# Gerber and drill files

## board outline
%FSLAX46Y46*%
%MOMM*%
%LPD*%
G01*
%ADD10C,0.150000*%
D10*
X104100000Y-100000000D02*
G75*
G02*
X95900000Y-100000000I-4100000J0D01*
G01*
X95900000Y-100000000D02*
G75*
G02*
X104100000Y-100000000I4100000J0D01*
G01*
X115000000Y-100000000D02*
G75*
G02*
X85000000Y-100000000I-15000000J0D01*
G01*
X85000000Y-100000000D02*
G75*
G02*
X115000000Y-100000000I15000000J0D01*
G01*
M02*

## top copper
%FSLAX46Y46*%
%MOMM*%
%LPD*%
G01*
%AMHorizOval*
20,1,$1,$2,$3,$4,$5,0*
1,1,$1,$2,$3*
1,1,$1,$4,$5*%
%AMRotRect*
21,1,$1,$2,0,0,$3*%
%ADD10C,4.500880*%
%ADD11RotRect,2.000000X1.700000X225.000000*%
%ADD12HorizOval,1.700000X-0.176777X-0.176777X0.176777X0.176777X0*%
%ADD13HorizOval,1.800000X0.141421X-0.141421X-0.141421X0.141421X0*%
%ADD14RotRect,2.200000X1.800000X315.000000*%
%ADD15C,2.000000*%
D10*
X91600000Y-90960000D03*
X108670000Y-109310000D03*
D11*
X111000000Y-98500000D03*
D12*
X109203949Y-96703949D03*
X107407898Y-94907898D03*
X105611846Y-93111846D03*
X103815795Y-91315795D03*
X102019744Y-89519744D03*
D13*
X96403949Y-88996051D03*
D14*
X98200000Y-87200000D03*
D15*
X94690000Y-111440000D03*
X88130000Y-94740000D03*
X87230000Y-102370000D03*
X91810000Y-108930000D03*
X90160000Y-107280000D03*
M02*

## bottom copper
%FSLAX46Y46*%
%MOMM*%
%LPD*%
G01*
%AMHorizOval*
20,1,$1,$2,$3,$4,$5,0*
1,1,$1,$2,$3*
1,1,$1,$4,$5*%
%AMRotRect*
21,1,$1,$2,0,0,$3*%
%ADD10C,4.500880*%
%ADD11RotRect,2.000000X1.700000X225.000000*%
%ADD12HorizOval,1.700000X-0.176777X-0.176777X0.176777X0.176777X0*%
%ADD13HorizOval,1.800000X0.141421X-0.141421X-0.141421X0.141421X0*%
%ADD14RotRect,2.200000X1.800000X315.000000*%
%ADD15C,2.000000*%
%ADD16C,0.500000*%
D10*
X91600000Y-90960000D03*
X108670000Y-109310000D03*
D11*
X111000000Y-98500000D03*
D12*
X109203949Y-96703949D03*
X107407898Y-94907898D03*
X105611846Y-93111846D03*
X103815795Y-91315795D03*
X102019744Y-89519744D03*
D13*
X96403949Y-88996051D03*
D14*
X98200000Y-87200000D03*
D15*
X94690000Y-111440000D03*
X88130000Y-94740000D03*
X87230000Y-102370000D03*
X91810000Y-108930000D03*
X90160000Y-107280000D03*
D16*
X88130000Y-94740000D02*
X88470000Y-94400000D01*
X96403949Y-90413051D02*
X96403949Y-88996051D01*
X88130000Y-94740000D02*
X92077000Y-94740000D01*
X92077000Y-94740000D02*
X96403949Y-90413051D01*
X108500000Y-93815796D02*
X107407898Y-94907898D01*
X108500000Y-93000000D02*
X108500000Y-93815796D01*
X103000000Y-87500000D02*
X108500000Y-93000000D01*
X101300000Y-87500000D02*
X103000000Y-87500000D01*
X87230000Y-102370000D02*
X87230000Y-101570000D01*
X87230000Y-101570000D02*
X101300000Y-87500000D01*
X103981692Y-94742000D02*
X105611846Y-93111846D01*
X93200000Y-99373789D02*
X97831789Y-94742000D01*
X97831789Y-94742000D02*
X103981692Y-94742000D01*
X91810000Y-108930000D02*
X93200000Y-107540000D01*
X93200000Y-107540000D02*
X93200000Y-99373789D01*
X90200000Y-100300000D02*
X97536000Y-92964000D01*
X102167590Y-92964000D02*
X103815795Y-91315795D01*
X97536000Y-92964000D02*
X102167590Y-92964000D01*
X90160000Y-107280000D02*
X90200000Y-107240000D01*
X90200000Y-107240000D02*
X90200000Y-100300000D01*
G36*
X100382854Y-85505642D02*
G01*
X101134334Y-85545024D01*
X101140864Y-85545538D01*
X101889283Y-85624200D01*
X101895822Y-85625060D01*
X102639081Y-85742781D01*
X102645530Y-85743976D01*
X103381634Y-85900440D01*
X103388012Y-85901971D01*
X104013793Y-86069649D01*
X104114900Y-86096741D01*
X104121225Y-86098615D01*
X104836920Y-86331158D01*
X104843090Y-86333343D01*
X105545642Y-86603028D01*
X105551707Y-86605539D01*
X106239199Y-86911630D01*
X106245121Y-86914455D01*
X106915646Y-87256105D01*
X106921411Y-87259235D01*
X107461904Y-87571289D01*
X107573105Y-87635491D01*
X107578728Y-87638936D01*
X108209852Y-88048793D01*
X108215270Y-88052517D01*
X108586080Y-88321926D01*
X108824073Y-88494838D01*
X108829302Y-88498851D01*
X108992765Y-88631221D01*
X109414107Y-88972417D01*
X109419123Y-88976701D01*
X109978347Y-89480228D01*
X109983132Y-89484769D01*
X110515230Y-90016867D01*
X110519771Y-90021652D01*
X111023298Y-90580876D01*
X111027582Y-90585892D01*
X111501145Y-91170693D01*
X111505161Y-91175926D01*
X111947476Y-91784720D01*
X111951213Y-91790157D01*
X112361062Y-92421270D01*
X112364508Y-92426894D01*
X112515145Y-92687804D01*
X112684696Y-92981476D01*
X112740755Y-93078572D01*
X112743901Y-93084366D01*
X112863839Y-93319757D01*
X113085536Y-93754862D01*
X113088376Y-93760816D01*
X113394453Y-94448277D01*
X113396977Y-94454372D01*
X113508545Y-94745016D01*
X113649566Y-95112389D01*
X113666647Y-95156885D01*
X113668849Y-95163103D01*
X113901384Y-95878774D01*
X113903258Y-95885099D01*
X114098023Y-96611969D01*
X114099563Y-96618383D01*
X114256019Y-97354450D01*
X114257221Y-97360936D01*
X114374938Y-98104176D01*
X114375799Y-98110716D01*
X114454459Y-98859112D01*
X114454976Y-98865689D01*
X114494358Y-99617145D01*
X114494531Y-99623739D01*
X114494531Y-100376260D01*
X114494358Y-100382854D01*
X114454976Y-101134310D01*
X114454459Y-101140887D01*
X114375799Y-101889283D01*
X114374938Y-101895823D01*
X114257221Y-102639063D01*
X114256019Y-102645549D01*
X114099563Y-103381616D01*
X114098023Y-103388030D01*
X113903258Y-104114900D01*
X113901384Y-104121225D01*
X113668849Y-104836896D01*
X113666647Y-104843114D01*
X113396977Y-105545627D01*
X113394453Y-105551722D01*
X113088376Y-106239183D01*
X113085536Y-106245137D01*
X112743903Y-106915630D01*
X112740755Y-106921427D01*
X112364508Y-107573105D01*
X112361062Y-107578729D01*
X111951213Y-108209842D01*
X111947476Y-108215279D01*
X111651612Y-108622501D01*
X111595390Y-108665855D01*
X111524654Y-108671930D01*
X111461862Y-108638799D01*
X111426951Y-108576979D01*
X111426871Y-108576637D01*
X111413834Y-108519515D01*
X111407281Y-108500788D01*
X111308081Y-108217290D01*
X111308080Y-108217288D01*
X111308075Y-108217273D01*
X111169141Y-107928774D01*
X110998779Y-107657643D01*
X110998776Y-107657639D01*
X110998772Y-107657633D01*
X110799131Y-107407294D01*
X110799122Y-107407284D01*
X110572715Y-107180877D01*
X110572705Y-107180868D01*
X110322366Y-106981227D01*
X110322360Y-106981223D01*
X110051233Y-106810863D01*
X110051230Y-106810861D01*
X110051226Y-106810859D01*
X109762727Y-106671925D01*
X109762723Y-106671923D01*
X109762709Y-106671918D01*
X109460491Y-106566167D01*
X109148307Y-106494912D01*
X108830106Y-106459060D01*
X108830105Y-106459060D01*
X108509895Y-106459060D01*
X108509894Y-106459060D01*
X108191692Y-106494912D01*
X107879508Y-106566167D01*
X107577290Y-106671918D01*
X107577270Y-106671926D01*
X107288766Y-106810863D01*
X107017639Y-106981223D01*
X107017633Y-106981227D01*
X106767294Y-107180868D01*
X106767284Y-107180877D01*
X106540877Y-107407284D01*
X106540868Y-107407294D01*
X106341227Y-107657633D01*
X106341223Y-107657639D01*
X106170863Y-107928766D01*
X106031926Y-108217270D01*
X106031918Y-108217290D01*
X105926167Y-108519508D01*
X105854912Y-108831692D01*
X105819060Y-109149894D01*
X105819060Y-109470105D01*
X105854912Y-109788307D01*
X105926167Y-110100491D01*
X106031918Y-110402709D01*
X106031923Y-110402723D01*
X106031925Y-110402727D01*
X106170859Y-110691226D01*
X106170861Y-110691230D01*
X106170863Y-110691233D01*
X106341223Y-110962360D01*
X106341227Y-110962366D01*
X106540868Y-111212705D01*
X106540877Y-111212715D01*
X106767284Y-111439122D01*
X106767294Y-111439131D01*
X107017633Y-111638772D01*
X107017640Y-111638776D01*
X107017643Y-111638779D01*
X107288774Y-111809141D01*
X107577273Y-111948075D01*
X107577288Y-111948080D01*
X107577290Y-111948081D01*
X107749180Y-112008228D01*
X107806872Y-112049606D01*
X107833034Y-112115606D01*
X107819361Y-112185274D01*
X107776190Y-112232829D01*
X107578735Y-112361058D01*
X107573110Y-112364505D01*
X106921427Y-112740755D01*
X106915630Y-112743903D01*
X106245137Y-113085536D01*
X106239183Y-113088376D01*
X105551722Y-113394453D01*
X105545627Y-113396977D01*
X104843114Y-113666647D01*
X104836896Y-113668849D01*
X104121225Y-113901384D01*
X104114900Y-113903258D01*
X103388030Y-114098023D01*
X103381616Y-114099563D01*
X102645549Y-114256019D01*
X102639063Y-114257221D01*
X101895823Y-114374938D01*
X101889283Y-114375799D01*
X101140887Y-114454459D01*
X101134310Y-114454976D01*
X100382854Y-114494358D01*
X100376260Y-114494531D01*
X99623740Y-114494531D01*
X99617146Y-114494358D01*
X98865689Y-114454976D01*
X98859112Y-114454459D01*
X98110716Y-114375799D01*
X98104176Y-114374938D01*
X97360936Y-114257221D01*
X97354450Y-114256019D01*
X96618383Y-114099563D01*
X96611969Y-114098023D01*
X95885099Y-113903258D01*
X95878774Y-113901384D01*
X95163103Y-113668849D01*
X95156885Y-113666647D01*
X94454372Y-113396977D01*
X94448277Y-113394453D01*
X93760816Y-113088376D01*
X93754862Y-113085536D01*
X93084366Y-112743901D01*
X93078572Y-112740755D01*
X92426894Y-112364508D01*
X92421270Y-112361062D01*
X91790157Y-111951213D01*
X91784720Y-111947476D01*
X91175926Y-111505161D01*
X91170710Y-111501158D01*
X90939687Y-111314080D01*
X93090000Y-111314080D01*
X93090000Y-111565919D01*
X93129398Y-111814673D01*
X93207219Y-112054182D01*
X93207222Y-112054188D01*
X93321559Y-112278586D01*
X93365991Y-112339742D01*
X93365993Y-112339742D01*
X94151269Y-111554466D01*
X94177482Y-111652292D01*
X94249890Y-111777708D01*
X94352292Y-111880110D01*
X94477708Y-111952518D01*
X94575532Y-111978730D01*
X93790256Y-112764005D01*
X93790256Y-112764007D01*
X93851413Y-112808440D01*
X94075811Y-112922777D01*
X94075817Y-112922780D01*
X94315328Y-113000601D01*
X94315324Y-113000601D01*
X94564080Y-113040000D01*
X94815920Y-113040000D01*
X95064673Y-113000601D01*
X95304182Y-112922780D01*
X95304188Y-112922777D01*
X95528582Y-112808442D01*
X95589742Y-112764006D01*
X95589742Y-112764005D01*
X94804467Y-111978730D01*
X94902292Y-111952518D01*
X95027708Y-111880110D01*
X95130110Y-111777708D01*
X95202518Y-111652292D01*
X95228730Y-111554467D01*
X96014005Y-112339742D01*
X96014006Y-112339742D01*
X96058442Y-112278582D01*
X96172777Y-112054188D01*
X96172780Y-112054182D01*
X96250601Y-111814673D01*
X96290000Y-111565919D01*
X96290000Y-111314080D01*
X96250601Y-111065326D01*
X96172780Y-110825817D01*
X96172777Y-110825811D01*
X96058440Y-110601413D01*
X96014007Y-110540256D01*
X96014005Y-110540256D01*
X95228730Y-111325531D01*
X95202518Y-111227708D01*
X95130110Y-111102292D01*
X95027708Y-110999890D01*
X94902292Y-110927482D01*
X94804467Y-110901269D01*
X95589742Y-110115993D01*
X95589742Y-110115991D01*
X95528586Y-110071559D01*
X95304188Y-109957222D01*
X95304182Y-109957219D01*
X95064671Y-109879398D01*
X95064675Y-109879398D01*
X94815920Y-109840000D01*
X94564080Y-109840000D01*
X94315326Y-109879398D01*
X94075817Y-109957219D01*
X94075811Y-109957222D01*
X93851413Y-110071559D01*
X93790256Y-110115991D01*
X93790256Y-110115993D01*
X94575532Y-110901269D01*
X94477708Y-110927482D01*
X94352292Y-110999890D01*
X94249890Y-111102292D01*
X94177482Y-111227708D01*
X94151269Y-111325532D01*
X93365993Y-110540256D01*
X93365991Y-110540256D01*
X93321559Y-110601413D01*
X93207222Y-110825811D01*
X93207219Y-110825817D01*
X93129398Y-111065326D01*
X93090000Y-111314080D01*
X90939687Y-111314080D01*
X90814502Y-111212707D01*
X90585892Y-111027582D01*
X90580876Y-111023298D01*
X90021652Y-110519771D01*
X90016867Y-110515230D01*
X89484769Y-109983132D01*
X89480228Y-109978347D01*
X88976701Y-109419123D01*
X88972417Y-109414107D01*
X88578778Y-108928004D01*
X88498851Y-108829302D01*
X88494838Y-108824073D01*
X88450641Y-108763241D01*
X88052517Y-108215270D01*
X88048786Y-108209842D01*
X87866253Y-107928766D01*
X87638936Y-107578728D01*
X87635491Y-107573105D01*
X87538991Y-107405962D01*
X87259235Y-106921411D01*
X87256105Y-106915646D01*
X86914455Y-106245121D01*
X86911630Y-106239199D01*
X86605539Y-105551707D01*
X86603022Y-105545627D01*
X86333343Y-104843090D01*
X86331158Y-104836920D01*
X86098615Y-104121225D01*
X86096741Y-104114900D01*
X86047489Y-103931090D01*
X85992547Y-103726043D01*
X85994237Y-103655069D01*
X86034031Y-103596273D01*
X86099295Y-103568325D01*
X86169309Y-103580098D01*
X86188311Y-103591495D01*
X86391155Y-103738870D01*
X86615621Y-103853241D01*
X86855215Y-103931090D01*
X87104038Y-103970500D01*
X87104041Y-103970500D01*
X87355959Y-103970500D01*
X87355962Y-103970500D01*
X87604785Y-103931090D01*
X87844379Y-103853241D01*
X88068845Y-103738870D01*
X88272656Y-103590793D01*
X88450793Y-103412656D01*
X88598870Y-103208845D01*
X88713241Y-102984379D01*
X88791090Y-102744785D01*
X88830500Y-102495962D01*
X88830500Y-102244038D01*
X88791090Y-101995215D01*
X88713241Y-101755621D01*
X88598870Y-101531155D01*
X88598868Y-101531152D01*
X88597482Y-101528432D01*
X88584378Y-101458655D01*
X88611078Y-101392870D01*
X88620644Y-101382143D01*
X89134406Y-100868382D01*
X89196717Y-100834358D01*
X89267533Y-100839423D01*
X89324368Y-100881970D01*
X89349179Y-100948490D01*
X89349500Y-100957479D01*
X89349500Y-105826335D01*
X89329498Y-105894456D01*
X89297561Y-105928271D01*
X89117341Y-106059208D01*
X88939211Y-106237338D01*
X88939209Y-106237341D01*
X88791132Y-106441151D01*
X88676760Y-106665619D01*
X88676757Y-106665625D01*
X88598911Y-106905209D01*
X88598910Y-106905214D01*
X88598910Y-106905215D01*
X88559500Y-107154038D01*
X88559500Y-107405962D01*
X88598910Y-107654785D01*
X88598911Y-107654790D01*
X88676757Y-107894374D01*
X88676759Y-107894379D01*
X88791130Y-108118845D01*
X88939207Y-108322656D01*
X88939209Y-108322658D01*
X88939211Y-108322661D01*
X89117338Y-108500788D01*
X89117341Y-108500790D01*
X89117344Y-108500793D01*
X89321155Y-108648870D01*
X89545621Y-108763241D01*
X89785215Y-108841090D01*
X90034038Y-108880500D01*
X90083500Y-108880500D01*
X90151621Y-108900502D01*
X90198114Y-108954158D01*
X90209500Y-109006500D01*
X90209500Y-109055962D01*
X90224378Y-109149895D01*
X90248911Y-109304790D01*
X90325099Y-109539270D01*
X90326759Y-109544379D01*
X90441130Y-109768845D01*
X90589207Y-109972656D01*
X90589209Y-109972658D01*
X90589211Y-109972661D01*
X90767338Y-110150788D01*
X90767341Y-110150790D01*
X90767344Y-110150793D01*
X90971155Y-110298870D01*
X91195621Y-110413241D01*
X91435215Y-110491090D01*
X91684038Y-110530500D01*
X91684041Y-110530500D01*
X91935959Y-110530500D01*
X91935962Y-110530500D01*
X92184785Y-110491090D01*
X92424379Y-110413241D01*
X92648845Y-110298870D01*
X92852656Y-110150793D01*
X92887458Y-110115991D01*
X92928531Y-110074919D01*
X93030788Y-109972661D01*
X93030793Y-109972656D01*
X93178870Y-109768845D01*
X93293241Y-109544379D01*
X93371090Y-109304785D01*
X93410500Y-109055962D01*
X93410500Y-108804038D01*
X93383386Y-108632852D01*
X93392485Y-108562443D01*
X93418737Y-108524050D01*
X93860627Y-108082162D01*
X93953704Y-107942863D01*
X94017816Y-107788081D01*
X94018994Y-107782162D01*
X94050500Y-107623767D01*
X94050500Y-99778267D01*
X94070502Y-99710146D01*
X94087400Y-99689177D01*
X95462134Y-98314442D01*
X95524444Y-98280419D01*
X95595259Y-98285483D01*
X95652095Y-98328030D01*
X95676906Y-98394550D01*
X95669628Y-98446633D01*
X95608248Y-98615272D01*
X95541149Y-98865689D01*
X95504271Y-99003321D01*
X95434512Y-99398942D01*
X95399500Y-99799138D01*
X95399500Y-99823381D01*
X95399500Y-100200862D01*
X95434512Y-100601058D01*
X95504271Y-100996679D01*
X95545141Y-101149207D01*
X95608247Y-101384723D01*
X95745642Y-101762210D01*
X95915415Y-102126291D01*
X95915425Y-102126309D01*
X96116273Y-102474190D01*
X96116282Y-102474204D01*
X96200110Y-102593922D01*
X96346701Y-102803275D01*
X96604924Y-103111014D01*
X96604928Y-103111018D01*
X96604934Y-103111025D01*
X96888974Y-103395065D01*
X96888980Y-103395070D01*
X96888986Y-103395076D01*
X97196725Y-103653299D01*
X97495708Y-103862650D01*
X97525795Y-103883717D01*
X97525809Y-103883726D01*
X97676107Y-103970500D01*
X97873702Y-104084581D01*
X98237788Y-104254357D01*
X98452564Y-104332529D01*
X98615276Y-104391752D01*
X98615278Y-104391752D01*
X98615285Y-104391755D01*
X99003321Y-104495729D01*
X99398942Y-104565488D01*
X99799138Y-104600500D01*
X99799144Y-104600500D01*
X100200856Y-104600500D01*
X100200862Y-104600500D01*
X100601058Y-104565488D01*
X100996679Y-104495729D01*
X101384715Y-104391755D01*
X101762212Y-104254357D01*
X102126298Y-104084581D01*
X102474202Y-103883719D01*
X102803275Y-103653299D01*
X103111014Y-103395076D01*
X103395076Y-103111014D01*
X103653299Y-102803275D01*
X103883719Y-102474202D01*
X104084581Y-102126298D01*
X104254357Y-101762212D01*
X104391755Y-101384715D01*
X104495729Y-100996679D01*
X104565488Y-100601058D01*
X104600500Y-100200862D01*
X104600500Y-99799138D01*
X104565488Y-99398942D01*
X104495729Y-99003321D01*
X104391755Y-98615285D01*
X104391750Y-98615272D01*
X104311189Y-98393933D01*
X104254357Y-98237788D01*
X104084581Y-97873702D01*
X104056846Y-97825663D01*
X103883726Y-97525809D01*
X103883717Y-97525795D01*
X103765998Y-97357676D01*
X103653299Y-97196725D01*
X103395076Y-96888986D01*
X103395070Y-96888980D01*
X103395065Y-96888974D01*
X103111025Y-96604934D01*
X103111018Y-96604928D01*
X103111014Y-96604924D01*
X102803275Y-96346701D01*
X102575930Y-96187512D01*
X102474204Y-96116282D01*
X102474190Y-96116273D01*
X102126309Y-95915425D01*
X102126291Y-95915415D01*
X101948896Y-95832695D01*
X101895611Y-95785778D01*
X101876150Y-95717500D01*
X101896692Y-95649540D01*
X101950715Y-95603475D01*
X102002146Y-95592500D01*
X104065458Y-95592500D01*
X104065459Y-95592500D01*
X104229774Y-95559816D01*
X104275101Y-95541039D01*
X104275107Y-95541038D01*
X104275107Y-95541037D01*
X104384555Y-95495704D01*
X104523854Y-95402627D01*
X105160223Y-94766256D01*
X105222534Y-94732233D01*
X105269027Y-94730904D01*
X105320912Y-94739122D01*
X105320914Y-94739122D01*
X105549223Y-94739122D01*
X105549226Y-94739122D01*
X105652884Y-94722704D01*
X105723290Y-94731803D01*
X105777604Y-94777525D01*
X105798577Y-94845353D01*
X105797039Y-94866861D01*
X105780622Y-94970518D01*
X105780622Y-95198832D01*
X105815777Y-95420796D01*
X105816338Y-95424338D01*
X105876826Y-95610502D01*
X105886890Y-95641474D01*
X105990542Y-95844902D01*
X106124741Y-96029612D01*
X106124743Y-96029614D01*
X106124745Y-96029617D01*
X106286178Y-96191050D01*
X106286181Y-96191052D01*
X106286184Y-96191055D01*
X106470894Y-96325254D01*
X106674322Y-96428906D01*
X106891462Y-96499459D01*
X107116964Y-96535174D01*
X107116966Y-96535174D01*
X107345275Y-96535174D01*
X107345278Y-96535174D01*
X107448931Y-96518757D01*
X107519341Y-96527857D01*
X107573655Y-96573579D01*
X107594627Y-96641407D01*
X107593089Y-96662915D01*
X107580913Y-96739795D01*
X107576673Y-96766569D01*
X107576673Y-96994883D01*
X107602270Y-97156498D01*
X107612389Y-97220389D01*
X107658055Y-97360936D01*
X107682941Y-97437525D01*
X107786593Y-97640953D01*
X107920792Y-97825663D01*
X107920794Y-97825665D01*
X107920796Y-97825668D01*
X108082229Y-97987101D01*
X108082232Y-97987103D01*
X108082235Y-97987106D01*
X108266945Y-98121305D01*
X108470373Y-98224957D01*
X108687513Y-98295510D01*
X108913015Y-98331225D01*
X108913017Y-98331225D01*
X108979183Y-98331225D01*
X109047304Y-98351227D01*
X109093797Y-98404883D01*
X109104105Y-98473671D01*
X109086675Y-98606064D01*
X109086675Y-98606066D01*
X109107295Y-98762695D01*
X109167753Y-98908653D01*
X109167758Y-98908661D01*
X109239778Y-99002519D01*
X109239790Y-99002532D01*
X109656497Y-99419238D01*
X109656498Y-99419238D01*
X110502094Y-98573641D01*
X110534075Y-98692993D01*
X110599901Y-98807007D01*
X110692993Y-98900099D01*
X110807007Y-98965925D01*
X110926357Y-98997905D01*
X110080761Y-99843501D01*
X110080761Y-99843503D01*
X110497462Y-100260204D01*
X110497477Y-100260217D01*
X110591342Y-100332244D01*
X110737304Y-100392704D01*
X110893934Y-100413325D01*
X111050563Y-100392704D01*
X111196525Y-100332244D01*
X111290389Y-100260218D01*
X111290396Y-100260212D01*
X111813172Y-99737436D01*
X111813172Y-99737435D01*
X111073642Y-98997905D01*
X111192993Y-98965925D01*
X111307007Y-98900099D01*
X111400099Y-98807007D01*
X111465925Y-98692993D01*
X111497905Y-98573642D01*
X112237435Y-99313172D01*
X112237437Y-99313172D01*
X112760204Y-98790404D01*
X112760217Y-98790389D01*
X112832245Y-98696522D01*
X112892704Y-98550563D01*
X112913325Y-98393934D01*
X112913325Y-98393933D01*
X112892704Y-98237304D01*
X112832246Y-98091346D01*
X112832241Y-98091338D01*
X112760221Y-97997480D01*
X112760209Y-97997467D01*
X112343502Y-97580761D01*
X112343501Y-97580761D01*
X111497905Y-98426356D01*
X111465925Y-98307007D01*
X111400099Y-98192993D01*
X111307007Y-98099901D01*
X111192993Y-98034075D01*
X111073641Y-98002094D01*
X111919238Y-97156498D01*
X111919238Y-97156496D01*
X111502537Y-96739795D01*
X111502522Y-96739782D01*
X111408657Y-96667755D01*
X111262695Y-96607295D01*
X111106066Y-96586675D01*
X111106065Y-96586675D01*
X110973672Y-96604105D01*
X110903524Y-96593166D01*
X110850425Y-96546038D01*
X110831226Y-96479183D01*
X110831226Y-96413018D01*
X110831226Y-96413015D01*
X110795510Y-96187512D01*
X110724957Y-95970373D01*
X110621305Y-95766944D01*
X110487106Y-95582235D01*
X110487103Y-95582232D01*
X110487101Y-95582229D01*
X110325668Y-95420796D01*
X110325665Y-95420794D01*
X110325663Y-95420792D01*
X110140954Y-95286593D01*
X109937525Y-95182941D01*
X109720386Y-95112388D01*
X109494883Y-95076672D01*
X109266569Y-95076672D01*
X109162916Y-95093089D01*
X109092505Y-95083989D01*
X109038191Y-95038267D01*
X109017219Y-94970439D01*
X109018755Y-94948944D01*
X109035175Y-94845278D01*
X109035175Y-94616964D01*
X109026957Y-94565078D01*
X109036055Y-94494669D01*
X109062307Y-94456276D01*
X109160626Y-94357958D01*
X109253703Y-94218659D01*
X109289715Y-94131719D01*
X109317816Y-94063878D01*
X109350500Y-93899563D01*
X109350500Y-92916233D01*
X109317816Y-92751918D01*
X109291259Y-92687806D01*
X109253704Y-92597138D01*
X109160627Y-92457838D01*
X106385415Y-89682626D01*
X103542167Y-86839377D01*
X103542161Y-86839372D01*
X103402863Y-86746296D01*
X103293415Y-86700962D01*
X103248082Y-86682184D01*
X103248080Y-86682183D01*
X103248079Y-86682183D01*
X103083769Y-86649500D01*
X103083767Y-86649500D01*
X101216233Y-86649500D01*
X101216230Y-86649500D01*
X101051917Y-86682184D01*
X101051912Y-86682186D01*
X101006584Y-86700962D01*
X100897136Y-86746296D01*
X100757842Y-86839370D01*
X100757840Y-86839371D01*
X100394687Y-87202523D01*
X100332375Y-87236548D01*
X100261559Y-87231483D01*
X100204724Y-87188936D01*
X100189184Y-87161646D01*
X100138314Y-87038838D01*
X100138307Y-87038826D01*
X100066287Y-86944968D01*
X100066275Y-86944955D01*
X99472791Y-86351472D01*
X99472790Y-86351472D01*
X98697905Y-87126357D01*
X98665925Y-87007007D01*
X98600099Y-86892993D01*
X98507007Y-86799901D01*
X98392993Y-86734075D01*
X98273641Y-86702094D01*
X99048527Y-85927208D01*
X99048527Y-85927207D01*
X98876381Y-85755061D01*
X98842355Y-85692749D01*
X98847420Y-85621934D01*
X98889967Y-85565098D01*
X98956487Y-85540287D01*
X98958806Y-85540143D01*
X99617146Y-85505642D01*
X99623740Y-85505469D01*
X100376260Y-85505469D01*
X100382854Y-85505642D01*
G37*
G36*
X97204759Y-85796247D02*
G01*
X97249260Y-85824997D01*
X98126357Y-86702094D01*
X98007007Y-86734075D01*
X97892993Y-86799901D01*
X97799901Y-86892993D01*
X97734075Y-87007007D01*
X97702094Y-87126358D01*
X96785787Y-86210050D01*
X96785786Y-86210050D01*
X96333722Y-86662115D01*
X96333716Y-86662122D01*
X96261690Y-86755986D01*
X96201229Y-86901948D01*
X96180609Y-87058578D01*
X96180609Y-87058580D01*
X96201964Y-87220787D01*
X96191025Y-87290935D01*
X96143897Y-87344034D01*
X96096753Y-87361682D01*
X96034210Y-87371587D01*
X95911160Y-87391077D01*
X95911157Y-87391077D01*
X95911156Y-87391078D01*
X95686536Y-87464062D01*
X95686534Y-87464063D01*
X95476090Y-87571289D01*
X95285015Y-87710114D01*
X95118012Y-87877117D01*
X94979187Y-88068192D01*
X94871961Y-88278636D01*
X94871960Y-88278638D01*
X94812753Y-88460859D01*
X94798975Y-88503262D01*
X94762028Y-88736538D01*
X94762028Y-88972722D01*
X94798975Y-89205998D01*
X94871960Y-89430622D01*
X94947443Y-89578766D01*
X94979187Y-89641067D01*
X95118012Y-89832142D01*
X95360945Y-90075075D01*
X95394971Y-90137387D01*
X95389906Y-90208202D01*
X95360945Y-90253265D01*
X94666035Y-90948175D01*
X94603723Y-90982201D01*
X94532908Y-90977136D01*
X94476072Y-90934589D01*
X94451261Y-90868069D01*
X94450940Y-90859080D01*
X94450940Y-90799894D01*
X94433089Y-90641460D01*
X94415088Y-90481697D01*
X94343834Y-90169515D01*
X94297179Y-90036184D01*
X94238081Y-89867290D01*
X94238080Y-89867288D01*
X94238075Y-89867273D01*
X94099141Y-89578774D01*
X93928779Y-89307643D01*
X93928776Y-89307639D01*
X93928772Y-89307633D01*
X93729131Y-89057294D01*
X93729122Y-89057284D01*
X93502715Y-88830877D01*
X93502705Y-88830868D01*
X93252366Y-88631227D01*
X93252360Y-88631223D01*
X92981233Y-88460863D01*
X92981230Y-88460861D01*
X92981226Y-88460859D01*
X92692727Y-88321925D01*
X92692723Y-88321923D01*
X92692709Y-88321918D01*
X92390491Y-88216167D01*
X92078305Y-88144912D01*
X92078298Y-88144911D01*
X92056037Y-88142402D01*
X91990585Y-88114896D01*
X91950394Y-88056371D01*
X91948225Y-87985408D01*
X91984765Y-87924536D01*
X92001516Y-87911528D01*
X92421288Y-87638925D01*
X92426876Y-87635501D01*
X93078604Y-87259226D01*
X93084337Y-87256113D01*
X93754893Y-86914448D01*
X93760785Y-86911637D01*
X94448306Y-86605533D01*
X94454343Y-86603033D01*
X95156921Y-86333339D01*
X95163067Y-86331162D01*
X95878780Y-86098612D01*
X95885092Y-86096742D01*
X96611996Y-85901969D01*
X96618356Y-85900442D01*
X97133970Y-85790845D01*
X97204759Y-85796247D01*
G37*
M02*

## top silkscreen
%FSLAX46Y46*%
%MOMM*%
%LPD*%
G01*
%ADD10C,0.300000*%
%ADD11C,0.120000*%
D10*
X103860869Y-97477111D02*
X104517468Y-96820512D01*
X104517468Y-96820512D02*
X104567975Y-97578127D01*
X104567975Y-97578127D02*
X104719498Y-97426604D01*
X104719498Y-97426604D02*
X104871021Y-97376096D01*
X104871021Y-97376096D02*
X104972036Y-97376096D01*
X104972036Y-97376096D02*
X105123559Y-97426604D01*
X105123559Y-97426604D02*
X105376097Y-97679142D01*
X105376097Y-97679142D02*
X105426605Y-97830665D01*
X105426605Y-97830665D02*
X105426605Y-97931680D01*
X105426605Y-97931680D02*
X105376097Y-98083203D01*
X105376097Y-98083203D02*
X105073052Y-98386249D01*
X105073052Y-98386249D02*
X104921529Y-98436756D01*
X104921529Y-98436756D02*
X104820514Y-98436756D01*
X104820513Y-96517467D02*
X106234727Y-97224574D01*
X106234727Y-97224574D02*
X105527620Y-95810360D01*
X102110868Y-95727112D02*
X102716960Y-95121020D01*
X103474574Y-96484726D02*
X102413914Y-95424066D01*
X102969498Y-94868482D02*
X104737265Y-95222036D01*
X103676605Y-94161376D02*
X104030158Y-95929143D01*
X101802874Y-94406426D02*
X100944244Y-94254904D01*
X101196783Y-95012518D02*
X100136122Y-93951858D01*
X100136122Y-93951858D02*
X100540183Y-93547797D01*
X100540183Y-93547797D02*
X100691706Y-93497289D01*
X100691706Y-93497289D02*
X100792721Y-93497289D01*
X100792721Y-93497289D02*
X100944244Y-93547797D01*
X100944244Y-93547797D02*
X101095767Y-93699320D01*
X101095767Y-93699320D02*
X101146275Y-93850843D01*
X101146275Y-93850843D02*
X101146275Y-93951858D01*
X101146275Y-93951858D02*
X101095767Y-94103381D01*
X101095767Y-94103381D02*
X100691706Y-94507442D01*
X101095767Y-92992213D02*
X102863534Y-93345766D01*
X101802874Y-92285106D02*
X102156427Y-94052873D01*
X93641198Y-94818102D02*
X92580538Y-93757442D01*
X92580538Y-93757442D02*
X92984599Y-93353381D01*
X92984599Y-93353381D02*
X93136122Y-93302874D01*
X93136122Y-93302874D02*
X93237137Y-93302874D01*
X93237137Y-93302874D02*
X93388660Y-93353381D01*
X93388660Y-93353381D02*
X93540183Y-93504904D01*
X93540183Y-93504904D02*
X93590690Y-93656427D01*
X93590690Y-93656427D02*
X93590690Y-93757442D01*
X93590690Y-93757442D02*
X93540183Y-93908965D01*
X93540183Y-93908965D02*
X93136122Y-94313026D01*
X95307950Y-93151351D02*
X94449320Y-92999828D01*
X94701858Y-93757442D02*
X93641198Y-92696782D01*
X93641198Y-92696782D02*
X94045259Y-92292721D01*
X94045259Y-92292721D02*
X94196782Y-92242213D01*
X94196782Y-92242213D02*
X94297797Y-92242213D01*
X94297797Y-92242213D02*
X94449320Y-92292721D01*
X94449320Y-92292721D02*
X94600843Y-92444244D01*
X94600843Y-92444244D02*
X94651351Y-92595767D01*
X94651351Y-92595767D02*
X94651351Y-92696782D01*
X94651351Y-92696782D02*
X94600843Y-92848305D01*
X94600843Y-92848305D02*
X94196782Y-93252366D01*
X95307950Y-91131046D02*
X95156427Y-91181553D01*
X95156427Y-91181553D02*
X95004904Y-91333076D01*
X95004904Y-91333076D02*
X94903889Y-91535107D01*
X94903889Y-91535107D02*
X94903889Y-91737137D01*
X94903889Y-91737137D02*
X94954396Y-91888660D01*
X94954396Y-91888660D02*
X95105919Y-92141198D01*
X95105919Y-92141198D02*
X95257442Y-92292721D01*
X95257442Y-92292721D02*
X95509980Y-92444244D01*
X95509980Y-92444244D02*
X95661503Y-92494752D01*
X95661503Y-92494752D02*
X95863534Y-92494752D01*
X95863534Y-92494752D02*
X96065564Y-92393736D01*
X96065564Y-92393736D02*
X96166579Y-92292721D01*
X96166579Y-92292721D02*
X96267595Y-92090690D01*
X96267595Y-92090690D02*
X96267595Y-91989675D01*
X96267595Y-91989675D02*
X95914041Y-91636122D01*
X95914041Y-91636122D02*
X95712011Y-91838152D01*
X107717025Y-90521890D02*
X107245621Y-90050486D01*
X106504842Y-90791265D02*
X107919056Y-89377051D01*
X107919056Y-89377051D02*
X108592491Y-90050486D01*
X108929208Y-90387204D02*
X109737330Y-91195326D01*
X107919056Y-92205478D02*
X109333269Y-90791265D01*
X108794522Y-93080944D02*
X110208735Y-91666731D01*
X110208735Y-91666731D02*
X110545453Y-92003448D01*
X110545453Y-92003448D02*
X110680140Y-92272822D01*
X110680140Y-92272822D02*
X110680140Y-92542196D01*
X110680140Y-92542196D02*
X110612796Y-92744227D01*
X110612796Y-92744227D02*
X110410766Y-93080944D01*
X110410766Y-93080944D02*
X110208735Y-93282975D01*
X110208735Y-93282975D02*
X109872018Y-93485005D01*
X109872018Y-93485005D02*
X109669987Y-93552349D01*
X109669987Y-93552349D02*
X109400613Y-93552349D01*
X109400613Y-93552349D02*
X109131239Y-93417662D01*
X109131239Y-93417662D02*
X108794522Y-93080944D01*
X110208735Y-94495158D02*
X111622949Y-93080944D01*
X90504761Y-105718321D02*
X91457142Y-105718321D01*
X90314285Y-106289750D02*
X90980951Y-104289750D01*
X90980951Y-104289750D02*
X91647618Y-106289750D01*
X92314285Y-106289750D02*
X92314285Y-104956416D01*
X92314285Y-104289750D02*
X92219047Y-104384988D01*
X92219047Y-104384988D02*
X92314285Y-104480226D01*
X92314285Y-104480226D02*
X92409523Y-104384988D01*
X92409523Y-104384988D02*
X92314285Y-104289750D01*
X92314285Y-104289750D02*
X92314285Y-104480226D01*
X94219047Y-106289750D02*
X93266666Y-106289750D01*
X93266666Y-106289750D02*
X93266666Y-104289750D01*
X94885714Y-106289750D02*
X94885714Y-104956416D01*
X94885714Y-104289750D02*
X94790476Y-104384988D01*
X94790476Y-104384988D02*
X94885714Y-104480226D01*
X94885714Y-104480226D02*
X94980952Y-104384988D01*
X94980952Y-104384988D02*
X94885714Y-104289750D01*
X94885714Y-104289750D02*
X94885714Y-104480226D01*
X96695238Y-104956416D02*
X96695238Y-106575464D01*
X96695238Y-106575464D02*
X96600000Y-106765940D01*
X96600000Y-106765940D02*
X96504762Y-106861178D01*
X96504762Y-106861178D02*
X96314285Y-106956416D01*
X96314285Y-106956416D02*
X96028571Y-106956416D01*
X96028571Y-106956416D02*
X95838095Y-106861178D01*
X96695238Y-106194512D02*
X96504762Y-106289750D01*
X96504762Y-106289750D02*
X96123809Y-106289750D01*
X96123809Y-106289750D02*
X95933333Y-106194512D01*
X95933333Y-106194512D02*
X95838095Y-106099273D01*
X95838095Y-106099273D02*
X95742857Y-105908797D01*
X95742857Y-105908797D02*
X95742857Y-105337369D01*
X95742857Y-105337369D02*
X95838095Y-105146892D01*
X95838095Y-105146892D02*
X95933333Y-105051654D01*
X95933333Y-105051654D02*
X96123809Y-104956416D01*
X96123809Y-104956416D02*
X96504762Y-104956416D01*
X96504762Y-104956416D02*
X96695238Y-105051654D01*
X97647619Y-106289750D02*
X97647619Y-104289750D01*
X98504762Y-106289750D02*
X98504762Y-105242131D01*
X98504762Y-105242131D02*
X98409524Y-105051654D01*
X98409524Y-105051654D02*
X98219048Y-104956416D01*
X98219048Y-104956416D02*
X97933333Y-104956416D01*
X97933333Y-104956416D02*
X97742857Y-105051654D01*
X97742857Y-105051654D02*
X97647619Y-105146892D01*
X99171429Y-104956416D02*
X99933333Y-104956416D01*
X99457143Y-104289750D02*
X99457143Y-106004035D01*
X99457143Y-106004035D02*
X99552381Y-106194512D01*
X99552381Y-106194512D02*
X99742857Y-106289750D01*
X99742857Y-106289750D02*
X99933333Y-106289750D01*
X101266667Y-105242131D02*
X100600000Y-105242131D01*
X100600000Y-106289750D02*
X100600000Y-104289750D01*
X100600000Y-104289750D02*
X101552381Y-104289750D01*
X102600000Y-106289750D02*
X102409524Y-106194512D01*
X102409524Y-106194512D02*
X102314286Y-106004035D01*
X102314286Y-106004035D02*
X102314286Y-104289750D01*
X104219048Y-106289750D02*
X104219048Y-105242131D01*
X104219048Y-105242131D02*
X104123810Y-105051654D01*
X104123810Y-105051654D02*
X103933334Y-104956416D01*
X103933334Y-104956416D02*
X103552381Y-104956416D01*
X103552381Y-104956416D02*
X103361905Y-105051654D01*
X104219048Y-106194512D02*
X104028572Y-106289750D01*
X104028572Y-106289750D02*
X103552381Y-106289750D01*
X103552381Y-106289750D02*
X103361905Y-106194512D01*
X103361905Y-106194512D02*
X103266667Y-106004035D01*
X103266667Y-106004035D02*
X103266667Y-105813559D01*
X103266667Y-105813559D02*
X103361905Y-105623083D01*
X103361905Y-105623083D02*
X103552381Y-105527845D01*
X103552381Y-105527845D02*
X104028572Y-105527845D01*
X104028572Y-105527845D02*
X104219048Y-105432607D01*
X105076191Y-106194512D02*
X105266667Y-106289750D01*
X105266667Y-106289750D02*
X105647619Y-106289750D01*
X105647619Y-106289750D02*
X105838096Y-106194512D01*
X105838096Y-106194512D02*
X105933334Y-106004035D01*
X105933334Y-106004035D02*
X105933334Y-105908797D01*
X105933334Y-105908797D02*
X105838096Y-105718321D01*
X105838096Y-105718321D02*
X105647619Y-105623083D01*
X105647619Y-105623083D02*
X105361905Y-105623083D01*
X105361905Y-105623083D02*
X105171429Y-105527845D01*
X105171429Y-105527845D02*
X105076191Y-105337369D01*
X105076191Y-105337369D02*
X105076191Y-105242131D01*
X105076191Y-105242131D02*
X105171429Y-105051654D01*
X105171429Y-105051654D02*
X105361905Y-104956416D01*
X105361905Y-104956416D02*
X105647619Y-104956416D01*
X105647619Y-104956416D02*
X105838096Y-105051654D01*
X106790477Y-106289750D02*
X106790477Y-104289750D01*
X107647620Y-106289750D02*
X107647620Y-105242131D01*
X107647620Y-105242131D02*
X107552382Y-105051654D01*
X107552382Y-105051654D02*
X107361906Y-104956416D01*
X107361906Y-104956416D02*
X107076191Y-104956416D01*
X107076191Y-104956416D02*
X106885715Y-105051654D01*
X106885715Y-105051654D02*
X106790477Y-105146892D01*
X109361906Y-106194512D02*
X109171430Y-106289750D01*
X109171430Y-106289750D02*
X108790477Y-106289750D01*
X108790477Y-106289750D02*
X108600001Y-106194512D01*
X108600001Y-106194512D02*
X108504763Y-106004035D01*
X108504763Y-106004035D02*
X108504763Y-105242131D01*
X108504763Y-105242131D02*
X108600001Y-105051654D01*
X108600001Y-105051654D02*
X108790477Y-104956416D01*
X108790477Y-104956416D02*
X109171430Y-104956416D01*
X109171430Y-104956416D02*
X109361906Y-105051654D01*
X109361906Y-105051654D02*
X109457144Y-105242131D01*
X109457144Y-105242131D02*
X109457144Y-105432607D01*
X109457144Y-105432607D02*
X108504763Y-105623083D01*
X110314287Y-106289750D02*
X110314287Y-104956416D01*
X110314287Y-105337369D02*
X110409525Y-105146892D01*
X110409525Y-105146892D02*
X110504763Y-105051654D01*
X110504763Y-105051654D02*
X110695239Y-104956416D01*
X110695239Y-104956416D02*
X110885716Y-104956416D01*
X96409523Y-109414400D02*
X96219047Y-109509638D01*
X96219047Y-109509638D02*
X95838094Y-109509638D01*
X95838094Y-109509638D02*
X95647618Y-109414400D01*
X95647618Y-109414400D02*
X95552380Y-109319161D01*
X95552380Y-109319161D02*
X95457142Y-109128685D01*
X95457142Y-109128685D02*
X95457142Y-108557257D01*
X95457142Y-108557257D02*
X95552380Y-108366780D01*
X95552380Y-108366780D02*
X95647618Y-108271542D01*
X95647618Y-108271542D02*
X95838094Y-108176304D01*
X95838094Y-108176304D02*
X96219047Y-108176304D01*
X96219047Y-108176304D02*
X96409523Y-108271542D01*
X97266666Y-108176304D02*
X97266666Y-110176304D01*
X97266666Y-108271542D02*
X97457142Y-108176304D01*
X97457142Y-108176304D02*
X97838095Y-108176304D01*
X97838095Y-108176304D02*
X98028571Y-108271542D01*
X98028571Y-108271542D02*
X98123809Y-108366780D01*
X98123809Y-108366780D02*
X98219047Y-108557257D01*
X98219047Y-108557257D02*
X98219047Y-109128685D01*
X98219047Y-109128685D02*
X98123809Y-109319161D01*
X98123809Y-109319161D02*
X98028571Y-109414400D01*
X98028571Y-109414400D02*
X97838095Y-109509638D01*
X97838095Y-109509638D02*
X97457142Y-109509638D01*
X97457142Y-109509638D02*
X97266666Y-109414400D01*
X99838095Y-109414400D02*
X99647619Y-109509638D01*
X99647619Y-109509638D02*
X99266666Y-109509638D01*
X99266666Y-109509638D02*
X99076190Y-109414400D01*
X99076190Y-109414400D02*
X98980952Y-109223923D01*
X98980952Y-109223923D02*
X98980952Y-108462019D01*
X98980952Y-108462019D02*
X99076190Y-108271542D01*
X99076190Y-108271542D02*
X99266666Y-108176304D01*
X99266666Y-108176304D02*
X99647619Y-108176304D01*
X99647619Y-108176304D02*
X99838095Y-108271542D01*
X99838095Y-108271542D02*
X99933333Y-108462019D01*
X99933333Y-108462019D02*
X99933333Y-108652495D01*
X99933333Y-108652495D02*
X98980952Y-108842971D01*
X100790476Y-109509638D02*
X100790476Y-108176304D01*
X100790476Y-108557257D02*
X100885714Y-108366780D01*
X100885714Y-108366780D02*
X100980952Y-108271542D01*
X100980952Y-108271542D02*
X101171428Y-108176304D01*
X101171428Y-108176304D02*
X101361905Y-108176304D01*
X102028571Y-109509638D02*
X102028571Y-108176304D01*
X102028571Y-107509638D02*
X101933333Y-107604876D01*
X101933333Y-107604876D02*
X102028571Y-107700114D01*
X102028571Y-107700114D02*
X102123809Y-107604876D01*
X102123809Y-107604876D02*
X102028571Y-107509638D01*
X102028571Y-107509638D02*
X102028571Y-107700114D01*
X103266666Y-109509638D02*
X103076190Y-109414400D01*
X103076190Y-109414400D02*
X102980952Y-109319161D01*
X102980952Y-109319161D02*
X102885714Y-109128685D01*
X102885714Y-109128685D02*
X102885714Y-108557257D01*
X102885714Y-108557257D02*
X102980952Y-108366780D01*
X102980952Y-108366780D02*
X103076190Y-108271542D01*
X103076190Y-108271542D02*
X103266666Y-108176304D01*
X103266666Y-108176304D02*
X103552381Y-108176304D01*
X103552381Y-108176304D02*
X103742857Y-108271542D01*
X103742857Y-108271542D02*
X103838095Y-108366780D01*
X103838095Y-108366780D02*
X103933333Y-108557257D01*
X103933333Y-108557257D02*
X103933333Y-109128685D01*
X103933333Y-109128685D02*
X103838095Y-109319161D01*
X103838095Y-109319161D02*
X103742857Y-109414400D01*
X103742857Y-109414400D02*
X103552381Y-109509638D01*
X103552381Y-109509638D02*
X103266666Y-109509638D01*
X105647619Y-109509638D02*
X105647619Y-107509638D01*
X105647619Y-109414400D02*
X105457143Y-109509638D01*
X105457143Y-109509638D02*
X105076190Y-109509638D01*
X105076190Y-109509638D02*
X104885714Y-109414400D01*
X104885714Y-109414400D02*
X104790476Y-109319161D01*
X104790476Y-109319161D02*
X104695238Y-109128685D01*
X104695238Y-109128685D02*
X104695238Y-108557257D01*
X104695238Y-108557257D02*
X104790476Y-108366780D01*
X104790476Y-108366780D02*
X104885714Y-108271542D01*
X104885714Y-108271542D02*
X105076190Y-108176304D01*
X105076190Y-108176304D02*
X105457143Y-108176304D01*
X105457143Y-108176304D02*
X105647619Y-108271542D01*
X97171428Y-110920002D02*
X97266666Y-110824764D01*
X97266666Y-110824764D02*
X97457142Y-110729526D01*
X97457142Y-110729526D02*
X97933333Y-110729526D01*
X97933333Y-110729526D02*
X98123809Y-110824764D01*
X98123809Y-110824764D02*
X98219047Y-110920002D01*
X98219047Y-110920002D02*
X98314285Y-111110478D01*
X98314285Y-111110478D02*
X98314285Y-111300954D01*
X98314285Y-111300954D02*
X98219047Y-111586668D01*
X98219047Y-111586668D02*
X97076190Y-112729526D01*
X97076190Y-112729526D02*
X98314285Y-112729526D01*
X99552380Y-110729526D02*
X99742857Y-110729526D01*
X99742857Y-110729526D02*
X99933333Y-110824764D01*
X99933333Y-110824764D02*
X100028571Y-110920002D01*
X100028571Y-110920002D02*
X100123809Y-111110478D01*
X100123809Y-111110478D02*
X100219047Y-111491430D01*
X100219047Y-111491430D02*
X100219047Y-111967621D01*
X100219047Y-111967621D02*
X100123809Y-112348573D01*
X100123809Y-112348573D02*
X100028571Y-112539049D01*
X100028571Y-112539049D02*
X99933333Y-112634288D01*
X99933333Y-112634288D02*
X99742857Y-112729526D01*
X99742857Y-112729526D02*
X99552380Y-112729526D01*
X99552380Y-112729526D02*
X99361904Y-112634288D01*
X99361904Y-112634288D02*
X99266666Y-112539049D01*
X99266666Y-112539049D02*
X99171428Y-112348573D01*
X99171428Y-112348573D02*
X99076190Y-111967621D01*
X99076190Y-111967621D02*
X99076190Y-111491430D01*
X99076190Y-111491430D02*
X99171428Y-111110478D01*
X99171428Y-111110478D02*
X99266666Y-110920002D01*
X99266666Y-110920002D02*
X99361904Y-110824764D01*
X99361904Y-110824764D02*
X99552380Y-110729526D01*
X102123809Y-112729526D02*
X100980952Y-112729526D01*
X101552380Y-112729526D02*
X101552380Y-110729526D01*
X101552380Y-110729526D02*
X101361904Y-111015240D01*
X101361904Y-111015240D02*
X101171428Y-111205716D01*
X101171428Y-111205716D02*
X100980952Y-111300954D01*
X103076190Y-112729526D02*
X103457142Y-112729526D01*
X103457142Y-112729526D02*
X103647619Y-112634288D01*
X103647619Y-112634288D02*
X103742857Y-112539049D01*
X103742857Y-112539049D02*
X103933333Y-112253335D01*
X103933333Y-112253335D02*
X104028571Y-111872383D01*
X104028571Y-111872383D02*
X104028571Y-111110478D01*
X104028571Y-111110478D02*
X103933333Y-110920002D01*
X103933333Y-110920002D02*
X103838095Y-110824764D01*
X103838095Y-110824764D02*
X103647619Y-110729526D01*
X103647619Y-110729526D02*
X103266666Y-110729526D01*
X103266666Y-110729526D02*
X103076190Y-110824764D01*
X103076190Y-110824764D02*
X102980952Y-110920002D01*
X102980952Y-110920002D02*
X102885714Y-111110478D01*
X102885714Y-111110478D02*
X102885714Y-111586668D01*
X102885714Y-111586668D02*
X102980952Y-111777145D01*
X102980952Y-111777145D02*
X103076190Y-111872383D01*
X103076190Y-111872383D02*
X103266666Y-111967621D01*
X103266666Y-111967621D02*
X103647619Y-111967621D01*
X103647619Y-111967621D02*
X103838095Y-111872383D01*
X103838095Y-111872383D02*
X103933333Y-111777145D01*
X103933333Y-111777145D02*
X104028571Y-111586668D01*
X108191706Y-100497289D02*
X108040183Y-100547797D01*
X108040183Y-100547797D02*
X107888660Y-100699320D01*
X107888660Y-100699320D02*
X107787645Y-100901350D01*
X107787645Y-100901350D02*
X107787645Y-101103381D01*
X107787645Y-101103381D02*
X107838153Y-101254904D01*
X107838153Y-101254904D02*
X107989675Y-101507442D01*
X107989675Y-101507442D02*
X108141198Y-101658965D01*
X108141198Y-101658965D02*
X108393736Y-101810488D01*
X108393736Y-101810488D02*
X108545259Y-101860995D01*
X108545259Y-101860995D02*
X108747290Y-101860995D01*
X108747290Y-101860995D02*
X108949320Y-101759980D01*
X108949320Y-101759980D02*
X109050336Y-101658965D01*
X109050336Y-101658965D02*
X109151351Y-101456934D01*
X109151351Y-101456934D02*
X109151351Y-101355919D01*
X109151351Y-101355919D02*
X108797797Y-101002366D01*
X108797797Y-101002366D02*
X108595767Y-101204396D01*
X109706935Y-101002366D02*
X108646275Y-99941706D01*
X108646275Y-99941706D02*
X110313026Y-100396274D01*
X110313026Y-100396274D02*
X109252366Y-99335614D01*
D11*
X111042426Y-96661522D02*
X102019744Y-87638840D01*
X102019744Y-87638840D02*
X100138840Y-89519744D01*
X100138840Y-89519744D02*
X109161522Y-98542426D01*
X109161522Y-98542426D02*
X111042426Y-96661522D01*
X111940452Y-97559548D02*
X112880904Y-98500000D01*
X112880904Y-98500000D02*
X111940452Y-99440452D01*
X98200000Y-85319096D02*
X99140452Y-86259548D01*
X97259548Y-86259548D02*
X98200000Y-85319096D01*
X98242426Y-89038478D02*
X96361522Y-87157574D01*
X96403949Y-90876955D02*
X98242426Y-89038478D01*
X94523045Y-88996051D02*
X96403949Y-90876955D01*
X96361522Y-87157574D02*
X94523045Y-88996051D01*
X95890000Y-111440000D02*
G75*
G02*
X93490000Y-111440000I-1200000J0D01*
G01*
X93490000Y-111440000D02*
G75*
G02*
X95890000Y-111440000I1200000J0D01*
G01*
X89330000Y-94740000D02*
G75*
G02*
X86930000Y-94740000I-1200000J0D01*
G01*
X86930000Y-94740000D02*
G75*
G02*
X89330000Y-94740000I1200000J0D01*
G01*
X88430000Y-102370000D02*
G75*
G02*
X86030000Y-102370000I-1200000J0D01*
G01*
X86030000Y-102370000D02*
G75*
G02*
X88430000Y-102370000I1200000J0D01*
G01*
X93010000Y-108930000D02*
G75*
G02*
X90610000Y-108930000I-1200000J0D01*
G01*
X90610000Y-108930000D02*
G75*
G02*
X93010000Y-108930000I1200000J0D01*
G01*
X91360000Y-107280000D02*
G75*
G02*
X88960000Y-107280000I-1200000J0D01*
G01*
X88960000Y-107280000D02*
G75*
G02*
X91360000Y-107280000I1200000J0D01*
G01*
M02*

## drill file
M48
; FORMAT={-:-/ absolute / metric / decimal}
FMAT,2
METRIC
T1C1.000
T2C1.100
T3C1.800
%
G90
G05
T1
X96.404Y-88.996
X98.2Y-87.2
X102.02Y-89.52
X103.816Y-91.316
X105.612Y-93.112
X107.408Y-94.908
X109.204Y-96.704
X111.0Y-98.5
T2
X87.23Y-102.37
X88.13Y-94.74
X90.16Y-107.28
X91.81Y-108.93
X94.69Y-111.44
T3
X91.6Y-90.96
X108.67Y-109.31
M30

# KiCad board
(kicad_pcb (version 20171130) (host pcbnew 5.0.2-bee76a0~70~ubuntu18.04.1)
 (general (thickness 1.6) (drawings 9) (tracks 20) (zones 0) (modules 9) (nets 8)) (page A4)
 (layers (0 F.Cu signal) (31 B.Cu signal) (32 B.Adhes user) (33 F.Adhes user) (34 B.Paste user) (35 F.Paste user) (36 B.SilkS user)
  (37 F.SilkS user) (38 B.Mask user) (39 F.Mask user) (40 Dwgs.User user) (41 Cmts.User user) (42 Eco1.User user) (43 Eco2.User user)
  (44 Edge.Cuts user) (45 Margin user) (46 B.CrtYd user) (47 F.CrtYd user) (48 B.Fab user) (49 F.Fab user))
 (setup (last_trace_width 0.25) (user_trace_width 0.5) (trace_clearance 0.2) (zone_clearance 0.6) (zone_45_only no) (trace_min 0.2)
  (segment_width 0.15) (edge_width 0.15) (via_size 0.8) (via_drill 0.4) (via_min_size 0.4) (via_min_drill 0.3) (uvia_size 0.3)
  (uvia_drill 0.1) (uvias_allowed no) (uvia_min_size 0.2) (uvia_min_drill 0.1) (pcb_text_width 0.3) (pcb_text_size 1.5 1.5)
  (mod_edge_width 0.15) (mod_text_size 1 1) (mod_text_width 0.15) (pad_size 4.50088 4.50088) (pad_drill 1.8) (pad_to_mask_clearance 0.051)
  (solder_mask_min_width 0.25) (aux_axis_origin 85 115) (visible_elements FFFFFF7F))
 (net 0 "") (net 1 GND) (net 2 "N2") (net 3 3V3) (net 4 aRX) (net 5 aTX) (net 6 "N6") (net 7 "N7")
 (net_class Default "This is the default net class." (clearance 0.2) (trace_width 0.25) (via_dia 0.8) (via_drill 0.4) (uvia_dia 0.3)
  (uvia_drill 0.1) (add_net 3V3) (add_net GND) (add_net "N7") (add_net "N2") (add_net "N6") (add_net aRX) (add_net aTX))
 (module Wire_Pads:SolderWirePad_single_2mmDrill (layer F.Cu) (at 91.6 90.96)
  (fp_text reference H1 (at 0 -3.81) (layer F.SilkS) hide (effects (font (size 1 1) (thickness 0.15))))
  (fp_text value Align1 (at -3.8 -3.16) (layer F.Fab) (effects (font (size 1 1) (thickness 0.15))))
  (pad 1 thru_hole circle (at 0 0) (size 4.50088 4.50088) (drill 1.8) (layers *.Cu *.Mask)))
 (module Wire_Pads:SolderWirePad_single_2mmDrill (layer F.Cu) (at 108.67 109.31)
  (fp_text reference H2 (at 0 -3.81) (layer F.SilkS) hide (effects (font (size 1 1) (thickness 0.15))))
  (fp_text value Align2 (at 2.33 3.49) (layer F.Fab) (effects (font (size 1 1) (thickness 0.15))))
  (pad 1 thru_hole circle (at 0 0) (size 4.50088 4.50088) (drill 1.8) (layers *.Cu *.Mask)))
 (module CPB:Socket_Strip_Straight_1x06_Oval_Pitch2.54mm (layer F.Cu) (at 111 98.5 225)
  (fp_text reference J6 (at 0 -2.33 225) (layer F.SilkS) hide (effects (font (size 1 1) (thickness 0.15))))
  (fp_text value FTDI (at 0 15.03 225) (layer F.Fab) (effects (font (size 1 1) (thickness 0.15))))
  (fp_line (start -1.33 1.27) (end -1.33 14.03) (layer F.SilkS) (width 0.12))
  (fp_line (start -1.33 14.03) (end 1.33 14.03) (layer F.SilkS) (width 0.12))
  (fp_line (start 1.33 14.03) (end 1.33 1.27) (layer F.SilkS) (width 0.12))
  (fp_line (start 1.33 1.27) (end -1.33 1.27) (layer F.SilkS) (width 0.12))
  (fp_line (start -1.33 0) (end -1.33 -1.33) (layer F.SilkS) (width 0.12))
  (fp_line (start -1.33 -1.33) (end 0 -1.33) (layer F.SilkS) (width 0.12))
  (pad 1 thru_hole rect (at 0 0 225) (size 2 1.7) (drill 1) (layers *.Cu *.Mask) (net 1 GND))
  (pad 2 thru_hole oval (at 0 2.54 225) (size 2.2 1.7) (drill 1) (layers *.Cu *.Mask) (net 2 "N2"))
  (pad 3 thru_hole oval (at 0 5.079999 225) (size 2.2 1.7) (drill 1) (layers *.Cu *.Mask) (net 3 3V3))
  (pad 4 thru_hole oval (at 0 7.62 225) (size 2.2 1.7) (drill 1) (layers *.Cu *.Mask) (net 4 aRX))
  (pad 5 thru_hole oval (at 0 10.16 225) (size 2.2 1.7) (drill 1) (layers *.Cu *.Mask) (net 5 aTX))
  (pad 6 thru_hole oval (at 0 12.7 225) (size 2.2 1.7) (drill 1) (layers *.Cu *.Mask) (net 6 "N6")))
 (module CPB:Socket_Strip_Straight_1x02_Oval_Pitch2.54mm (layer F.Cu) (at 98.2 87.2 315)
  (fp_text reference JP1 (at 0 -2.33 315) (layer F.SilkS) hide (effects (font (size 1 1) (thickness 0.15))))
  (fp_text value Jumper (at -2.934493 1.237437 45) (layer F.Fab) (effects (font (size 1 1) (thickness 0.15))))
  (fp_line (start -1.33 -1.33) (end 0 -1.33) (layer F.SilkS) (width 0.12))
  (fp_line (start -1.33 0) (end -1.33 -1.33) (layer F.SilkS) (width 0.12))
  (fp_line (start 1.33 1.27) (end -1.33 1.27) (layer F.SilkS) (width 0.12))
  (fp_line (start 1.33 3.87) (end 1.33 1.27) (layer F.SilkS) (width 0.12))
  (fp_line (start -1.33 3.87) (end 1.33 3.87) (layer F.SilkS) (width 0.12))
  (fp_line (start -1.33 1.27) (end -1.33 3.87) (layer F.SilkS) (width 0.12))
  (pad 2 thru_hole oval (at 0 2.54 315) (size 2.2 1.8) (drill 1) (layers *.Cu *.Mask) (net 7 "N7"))
  (pad 1 thru_hole rect (at 0 0 315) (size 2.2 1.8) (drill 1) (layers *.Cu *.Mask) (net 1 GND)))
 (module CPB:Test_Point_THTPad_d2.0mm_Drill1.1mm (layer F.Cu) (at 94.69 111.44)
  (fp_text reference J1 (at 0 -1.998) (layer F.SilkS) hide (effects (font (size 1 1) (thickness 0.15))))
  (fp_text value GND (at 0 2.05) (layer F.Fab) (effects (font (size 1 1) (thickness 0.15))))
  (fp_circle (center 0 0) (end 0 1.2) (layer F.SilkS) (width 0.12))
  (pad 1 thru_hole circle (at 0 0) (size 2 2) (drill 1.1) (layers *.Cu *.Mask) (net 1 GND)))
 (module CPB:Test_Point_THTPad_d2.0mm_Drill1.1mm (layer F.Cu) (at 88.13 94.74)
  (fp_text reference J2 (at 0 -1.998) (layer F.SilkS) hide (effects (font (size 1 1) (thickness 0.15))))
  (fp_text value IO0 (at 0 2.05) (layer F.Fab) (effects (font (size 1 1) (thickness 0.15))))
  (fp_circle (center 0 0) (end 0 1.2) (layer F.SilkS) (width 0.12))
  (pad 1 thru_hole circle (at 0 0) (size 2 2) (drill 1.1) (layers *.Cu *.Mask) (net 7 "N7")))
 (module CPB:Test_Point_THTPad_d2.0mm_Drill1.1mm (layer F.Cu) (at 87.23 102.37)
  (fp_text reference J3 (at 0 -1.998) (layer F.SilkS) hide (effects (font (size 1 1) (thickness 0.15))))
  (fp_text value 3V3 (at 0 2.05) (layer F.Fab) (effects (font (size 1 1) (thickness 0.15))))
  (fp_circle (center 0 0) (end 0 1.2) (layer F.SilkS) (width 0.12))
  (pad 1 thru_hole circle (at 0 0) (size 2 2) (drill 1.1) (layers *.Cu *.Mask) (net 3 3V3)))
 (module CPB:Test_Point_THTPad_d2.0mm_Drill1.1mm (layer F.Cu) (at 91.81 108.93)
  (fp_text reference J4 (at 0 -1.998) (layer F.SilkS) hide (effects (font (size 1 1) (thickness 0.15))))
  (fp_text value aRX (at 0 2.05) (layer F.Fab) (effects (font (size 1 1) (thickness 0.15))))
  (fp_circle (center 0 0) (end 0 1.2) (layer F.SilkS) (width 0.12))
  (pad 1 thru_hole circle (at 0 0) (size 2 2) (drill 1.1) (layers *.Cu *.Mask) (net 4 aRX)))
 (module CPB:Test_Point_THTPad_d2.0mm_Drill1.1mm (layer F.Cu) (at 90.16 107.28)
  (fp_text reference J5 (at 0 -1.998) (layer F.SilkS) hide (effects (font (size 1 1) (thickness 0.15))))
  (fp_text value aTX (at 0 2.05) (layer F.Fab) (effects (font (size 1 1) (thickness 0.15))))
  (fp_circle (center 0 0) (end 0 1.2) (layer F.SilkS) (width 0.12))
  (pad 1 thru_hole circle (at 0 0) (size 2 2) (drill 1.1) (layers *.Cu *.Mask) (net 5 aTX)))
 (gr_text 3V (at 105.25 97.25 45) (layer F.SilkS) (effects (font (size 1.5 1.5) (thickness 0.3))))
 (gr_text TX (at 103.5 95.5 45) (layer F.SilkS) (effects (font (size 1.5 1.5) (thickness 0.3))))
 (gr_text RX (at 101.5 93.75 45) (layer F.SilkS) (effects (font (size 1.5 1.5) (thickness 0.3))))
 (gr_circle (center 100 100) (end 104.1 100) (layer Edge.Cuts) (width 0.15))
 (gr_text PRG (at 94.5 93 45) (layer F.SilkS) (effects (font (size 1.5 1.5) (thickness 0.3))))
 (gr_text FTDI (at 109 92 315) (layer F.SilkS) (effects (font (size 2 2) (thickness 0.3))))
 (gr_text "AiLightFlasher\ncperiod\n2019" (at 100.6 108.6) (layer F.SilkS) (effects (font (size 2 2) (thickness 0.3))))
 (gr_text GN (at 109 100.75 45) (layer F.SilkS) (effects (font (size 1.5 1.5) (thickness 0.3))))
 (gr_circle (center 100 100) (end 115 100) (layer Edge.Cuts) (width 0.15))
 (segment (start 88.13 94.74) (end 88.47 94.4) (width 0.5) (layer B.Cu) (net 7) (status 30))
 (segment (start 96.403949 90.413051) (end 96.403949 88.996051) (width 0.5) (layer B.Cu) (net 7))
 (segment (start 88.13 94.74) (end 92.077 94.74) (width 0.5) (layer B.Cu) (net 7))
 (segment (start 92.077 94.74) (end 96.403949 90.413051) (width 0.5) (layer B.Cu) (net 7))
 (segment (start 108.5 93.815796) (end 107.407898 94.907898) (width 0.5) (layer B.Cu) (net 3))
 (segment (start 108.5 93) (end 108.5 93.815796) (width 0.5) (layer B.Cu) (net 3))
 (segment (start 103 87.5) (end 108.5 93) (width 0.5) (layer B.Cu) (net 3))
 (segment (start 101.3 87.5) (end 103 87.5) (width 0.5) (layer B.Cu) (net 3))
 (segment (start 87.23 102.37) (end 87.23 101.57) (width 0.5) (layer B.Cu) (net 3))
 (segment (start 87.23 101.57) (end 101.3 87.5) (width 0.5) (layer B.Cu) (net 3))
 (segment (start 103.981692 94.742) (end 105.611846 93.111846) (width 0.5) (layer B.Cu) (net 4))
 (segment (start 93.2 99.373789) (end 97.831789 94.742) (width 0.5) (layer B.Cu) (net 4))
 (segment (start 97.831789 94.742) (end 103.981692 94.742) (width 0.5) (layer B.Cu) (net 4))
 (segment (start 91.81 108.93) (end 93.2 107.54) (width 0.5) (layer B.Cu) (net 4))
 (segment (start 93.2 107.54) (end 93.2 99.373789) (width 0.5) (layer B.Cu) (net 4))
 (segment (start 90.2 100.3) (end 97.536 92.964) (width 0.5) (layer B.Cu) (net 5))
 (segment (start 102.16759 92.964) (end 103.815795 91.315795) (width 0.5) (layer B.Cu) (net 5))
 (segment (start 97.536 92.964) (end 102.16759 92.964) (width 0.5) (layer B.Cu) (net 5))
 (segment (start 90.16 107.28) (end 90.2 107.24) (width 0.5) (layer B.Cu) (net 5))
 (segment (start 90.2 107.24) (end 90.2 100.3) (width 0.5) (layer B.Cu) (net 5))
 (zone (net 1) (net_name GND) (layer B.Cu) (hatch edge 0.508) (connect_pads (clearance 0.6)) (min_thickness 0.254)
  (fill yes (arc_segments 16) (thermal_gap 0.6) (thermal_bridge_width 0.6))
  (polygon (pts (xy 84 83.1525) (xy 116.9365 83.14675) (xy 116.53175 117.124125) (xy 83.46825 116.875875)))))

